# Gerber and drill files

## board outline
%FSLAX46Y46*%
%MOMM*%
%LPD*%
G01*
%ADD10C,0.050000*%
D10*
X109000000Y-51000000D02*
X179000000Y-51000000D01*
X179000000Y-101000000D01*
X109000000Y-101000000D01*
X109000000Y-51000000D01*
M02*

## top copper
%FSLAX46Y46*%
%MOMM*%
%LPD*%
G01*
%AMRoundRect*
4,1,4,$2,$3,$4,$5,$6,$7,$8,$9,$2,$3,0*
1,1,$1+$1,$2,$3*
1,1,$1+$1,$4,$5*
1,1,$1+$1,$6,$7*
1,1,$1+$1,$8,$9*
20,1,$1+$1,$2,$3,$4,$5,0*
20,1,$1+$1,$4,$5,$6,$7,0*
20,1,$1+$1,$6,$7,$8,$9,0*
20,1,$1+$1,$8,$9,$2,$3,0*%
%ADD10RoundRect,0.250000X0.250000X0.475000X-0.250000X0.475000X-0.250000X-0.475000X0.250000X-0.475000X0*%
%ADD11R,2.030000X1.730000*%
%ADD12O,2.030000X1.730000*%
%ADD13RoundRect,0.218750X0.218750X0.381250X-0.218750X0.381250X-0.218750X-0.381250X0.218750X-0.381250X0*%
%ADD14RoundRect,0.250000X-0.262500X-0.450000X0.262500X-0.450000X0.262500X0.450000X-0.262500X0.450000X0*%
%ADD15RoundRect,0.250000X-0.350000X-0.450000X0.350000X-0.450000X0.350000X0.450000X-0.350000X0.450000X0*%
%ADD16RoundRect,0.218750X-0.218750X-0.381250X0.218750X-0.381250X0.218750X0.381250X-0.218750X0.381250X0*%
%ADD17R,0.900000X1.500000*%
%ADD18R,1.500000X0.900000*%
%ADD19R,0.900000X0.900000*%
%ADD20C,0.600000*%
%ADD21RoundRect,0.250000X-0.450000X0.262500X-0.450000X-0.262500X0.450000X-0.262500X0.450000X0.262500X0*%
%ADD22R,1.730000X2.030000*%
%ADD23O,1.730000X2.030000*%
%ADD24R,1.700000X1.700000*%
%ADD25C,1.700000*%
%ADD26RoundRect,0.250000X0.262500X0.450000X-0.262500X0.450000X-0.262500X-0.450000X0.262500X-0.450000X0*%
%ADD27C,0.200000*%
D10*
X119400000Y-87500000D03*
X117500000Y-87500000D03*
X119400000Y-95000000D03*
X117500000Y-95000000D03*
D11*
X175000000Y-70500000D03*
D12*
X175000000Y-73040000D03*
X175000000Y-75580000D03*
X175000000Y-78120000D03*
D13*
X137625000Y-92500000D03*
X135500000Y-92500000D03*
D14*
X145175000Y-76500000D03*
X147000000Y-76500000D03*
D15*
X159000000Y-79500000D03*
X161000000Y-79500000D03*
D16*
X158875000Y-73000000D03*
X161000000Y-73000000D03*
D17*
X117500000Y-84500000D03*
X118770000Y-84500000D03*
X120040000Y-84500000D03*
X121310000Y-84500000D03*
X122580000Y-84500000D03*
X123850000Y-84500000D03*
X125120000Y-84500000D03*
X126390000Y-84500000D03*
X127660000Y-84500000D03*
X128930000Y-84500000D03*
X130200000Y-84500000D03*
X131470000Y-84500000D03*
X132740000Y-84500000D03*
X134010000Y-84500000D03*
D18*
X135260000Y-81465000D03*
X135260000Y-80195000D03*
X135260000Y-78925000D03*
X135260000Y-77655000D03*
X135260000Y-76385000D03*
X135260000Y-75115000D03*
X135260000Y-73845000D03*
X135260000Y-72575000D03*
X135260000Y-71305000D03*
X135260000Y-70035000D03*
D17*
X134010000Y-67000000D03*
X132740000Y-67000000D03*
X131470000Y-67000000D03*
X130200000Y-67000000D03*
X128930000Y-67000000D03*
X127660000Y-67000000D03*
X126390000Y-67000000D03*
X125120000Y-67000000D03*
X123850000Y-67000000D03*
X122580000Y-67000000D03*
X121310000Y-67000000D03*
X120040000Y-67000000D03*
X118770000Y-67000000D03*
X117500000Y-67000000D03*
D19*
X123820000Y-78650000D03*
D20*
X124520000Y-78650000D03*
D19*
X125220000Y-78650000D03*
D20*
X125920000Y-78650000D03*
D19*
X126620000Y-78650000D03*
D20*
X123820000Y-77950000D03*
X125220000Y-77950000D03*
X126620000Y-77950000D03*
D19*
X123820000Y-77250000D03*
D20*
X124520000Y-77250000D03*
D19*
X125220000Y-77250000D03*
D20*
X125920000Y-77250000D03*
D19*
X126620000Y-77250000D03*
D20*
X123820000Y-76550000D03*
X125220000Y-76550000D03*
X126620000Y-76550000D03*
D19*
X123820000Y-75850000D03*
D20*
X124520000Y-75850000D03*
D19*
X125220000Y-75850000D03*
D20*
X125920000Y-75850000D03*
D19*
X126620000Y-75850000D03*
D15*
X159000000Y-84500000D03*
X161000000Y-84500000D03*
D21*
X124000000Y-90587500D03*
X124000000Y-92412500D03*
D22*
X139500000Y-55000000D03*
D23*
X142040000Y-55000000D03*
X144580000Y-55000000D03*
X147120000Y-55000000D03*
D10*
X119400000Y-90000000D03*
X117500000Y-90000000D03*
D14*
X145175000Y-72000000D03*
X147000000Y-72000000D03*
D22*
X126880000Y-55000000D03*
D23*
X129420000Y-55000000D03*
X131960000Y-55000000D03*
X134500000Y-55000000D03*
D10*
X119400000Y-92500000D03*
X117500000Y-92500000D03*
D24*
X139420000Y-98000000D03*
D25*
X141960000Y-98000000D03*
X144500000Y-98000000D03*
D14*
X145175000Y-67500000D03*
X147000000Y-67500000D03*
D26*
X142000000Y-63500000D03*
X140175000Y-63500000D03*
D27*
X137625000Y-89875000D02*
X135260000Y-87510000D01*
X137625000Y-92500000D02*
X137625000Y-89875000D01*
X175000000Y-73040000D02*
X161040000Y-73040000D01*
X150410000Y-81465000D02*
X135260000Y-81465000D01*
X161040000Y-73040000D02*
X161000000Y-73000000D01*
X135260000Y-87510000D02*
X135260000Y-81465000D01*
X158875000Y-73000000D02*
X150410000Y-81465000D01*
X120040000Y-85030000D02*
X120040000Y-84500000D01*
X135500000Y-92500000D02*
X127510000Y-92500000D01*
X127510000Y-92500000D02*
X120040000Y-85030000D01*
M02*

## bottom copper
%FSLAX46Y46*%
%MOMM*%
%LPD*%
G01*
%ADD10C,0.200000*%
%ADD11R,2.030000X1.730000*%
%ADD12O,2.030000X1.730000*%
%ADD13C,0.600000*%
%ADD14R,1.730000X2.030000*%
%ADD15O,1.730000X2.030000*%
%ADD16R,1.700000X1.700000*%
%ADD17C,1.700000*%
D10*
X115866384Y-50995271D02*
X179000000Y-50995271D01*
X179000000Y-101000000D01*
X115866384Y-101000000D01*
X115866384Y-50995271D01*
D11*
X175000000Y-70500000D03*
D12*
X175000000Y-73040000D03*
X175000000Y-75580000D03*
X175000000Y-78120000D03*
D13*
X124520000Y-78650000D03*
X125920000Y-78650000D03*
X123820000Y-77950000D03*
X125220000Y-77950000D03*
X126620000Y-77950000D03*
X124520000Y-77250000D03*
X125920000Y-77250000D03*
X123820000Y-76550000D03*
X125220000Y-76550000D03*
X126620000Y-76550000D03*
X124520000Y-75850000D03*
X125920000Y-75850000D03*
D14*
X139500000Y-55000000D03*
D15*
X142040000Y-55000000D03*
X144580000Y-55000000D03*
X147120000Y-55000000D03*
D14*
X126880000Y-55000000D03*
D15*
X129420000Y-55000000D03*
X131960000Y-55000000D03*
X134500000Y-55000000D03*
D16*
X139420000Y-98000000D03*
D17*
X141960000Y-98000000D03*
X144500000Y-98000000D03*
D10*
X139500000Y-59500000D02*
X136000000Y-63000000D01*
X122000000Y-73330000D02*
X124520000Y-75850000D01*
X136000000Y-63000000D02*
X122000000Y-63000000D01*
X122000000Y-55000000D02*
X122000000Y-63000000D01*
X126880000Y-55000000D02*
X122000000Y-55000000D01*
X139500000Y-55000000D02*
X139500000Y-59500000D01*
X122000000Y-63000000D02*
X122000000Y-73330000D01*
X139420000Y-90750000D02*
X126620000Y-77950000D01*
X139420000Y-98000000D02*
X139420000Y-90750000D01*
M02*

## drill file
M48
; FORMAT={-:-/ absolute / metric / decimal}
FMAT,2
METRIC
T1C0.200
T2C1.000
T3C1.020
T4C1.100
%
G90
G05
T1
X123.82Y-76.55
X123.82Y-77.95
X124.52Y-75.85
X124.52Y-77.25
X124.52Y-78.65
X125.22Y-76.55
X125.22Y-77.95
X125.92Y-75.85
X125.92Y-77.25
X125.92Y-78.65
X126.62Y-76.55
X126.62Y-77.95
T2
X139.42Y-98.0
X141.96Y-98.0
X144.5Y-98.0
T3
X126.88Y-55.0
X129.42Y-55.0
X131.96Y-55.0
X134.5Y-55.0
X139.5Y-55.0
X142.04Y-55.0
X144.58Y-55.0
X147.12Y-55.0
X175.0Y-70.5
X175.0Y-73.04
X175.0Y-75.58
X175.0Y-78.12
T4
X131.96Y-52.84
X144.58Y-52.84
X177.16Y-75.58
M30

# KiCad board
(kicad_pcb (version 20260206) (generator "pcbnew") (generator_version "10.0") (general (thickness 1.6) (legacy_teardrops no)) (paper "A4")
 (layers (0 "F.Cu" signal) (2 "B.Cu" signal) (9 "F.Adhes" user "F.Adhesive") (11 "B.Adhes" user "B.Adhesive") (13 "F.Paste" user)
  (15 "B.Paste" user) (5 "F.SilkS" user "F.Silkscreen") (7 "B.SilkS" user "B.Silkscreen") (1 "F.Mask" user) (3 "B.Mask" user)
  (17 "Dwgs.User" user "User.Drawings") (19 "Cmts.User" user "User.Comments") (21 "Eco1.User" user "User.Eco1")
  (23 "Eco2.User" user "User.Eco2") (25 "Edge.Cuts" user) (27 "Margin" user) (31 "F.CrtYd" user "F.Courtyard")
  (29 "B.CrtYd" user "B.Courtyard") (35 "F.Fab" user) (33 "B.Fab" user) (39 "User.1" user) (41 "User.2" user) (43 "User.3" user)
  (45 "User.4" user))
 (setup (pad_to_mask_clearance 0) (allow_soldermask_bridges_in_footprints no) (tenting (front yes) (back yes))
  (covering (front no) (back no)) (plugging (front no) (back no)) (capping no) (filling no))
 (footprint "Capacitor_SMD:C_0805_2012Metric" (layer "F.Cu") (at 118.45 87.5 180)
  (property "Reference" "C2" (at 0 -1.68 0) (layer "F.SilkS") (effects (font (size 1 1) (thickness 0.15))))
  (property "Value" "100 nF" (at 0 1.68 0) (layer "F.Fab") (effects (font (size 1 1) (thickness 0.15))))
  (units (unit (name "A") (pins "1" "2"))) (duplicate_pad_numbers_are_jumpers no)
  (pad "1" smd roundrect (at -0.95 0 180) (size 1 1.45) (layers "F.Cu" "F.Mask" "F.Paste") (roundrect_rratio 0.25) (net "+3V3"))
  (pad "2" smd roundrect (at 0.95 0 180) (size 1 1.45) (layers "F.Cu" "F.Mask" "F.Paste") (roundrect_rratio 0.25) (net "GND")))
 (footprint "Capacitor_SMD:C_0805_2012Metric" (layer "F.Cu") (at 118.45 95 180)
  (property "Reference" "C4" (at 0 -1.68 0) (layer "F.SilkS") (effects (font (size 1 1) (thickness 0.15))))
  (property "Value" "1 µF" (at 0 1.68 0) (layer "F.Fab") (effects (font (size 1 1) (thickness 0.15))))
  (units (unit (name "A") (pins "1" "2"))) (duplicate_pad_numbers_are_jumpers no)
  (pad "1" smd roundrect (at -0.95 0 180) (size 1 1.45) (layers "F.Cu" "F.Mask" "F.Paste") (roundrect_rratio 0.25) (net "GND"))
  (pad "2" smd roundrect (at 0.95 0 180) (size 1 1.45) (layers "F.Cu" "F.Mask" "F.Paste") (roundrect_rratio 0.25) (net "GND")))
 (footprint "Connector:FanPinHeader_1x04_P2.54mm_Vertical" (layer "F.Cu") (at 175 70.5 -90)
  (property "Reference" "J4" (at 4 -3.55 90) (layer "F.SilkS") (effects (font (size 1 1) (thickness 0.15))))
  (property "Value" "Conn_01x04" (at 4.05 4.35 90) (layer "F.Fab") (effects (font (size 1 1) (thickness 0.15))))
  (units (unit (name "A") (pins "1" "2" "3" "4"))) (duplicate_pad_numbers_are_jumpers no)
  (pad "" np_thru_hole circle (at 5.08 -2.16) (size 1.1 1.1) (drill 1.1) (layers "*.Cu" "*.Mask"))
  (pad "1" thru_hole rect (at 0 0) (size 2.03 1.73) (drill 1.02) (layers "*.Cu" "*.Mask") (remove_unused_layers no) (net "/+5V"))
  (pad "2" thru_hole oval (at 2.54 0) (size 2.03 1.73) (drill 1.02) (layers "*.Cu" "*.Mask") (remove_unused_layers no) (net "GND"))
  (pad "3" thru_hole oval (at 5.08 0) (size 2.03 1.73) (drill 1.02) (layers "*.Cu" "*.Mask") (remove_unused_layers no)
   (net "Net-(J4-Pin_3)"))
  (pad "4" thru_hole oval (at 7.62 0) (size 2.03 1.73) (drill 1.02) (layers "*.Cu" "*.Mask") (remove_unused_layers no) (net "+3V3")))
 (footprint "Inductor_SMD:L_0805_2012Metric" (layer "F.Cu") (at 136.5625 92.5 180)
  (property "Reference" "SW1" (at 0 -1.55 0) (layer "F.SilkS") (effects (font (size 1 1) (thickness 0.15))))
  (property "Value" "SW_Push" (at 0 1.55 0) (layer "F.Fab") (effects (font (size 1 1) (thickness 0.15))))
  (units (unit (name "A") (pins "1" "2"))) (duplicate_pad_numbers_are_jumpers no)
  (pad "1" smd roundrect (at -1.0625 0 180) (size 0.875 1.2) (layers "F.Cu" "F.Mask" "F.Paste") (roundrect_rratio 0.25) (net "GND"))
  (pad "2" smd roundrect (at 1.0625 0 180) (size 0.875 1.2) (layers "F.Cu" "F.Mask" "F.Paste") (roundrect_rratio 0.25) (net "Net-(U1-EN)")))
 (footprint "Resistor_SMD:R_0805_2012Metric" (layer "F.Cu") (at 146.0875 76.5)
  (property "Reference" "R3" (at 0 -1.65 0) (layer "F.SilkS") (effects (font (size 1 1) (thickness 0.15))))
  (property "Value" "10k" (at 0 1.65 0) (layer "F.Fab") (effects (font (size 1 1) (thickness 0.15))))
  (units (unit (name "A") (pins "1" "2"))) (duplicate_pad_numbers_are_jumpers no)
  (pad "1" smd roundrect (at -0.9125 0) (size 1.025 1.4) (layers "F.Cu" "F.Mask" "F.Paste") (roundrect_rratio 0.243902) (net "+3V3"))
  (pad "2" smd roundrect (at 0.9125 0) (size 1.025 1.4) (layers "F.Cu" "F.Mask" "F.Paste") (roundrect_rratio 0.243902) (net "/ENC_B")))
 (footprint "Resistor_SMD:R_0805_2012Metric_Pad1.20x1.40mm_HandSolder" (layer "F.Cu") (at 160 79.5)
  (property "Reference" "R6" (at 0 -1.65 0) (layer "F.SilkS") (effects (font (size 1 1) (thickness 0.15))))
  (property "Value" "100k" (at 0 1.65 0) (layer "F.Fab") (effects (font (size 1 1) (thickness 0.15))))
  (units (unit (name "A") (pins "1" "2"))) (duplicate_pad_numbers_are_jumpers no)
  (pad "1" smd roundrect (at -1 0) (size 1.2 1.4) (layers "F.Cu" "F.Mask" "F.Paste") (roundrect_rratio 0.208333) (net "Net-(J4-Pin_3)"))
  (pad "2" smd roundrect (at 1 0) (size 1.2 1.4) (layers "F.Cu" "F.Mask" "F.Paste") (roundrect_rratio 0.208333) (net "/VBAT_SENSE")))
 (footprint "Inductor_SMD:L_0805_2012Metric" (layer "F.Cu") (at 159.9375 73)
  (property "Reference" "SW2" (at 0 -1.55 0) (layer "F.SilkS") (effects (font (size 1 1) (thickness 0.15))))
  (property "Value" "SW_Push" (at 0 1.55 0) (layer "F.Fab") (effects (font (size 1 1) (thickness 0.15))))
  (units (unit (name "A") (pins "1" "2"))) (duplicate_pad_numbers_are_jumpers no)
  (pad "1" smd roundrect (at -1.0625 0) (size 0.875 1.2) (layers "F.Cu" "F.Mask" "F.Paste") (roundrect_rratio 0.25) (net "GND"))
  (pad "2" smd roundrect (at 1.0625 0) (size 0.875 1.2) (layers "F.Cu" "F.Mask" "F.Paste") (roundrect_rratio 0.25) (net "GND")))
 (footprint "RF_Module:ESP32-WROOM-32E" (layer "F.Cu") (at 122.76 75.75 90)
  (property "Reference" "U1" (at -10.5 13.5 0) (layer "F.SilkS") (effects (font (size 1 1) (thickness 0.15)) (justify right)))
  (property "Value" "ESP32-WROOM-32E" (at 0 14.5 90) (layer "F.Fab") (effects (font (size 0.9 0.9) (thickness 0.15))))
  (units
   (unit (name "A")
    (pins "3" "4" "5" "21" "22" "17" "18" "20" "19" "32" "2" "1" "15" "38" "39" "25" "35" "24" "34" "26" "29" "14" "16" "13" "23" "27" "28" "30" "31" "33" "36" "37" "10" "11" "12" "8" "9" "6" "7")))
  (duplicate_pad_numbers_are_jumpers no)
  (pad "1" smd rect (at -8.75 -5.26 90) (size 1.5 0.9) (layers "F.Cu" "F.Mask" "F.Paste") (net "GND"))
  (pad "2" smd rect (at -8.75 -3.99 90) (size 1.5 0.9) (layers "F.Cu" "F.Mask" "F.Paste") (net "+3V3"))
  (pad "3" smd rect (at -8.75 -2.72 90) (size 1.5 0.9) (layers "F.Cu" "F.Mask" "F.Paste") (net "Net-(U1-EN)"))
  (pad "4" smd rect (at -8.75 -1.45 90) (size 1.5 0.9) (layers "F.Cu" "F.Mask" "F.Paste") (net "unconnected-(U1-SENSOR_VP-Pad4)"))
  (pad "5" smd rect (at -8.75 -0.18 90) (size 1.5 0.9) (layers "F.Cu" "F.Mask" "F.Paste") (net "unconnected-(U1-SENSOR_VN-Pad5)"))
  (pad "6" smd rect (at -8.75 1.09 90) (size 1.5 0.9) (layers "F.Cu" "F.Mask" "F.Paste") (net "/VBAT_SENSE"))
  (pad "7" smd rect (at -8.75 2.36 90) (size 1.5 0.9) (layers "F.Cu" "F.Mask" "F.Paste") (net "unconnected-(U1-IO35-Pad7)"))
  (pad "8" smd rect (at -8.75 3.63 90) (size 1.5 0.9) (layers "F.Cu" "F.Mask" "F.Paste") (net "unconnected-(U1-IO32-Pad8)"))
  (pad "9" smd rect (at -8.75 4.9 90) (size 1.5 0.9) (layers "F.Cu" "F.Mask" "F.Paste") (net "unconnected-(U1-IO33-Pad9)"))
  (pad "10" smd rect (at -8.75 6.17 90) (size 1.5 0.9) (layers "F.Cu" "F.Mask" "F.Paste") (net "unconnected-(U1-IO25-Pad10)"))
  (pad "11" smd rect (at -8.75 7.44 90) (size 1.5 0.9) (layers "F.Cu" "F.Mask" "F.Paste") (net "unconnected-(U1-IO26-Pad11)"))
  (pad "12" smd rect (at -8.75 8.71 90) (size 1.5 0.9) (layers "F.Cu" "F.Mask" "F.Paste") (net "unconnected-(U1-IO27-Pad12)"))
  (pad "13" smd rect (at -8.75 9.98 90) (size 1.5 0.9) (layers "F.Cu" "F.Mask" "F.Paste") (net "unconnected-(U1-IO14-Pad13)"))
  (pad "14" smd rect (at -8.75 11.25 90) (size 1.5 0.9) (layers "F.Cu" "F.Mask" "F.Paste") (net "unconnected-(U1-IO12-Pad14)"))
  (pad "15" smd rect (at -5.715 12.5 180) (size 1.5 0.9) (layers "F.Cu" "F.Mask" "F.Paste") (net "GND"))
  (pad "16" smd rect (at -4.445 12.5 180) (size 1.5 0.9) (layers "F.Cu" "F.Mask" "F.Paste") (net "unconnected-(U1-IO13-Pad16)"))
  (pad "17" smd rect (at -3.175 12.5 180) (size 1.5 0.9) (layers "F.Cu" "F.Mask" "F.Paste") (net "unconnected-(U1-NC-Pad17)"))
  (pad "18" smd rect (at -1.905 12.5 180) (size 1.5 0.9) (layers "F.Cu" "F.Mask" "F.Paste") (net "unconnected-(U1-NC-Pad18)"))
  (pad "19" smd rect (at -0.635 12.5 180) (size 1.5 0.9) (layers "F.Cu" "F.Mask" "F.Paste") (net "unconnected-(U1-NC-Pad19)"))
  (pad "20" smd rect (at 0.635 12.5 180) (size 1.5 0.9) (layers "F.Cu" "F.Mask" "F.Paste") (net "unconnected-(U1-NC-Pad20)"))
  (pad "21" smd rect (at 1.905 12.5 180) (size 1.5 0.9) (layers "F.Cu" "F.Mask" "F.Paste") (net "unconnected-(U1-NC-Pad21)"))
  (pad "22" smd rect (at 3.175 12.5 180) (size 1.5 0.9) (layers "F.Cu" "F.Mask" "F.Paste") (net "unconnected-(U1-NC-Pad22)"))
  (pad "23" smd rect (at 4.445 12.5 180) (size 1.5 0.9) (layers "F.Cu" "F.Mask" "F.Paste") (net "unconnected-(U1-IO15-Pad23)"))
  (pad "24" smd rect (at 5.715 12.5 180) (size 1.5 0.9) (layers "F.Cu" "F.Mask" "F.Paste") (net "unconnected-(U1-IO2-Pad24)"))
  (pad "25" smd rect (at 8.75 11.25 90) (size 1.5 0.9) (layers "F.Cu" "F.Mask" "F.Paste") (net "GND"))
  (pad "26" smd rect (at 8.75 9.98 90) (size 1.5 0.9) (layers "F.Cu" "F.Mask" "F.Paste") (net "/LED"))
  (pad "27" smd rect (at 8.75 8.71 90) (size 1.5 0.9) (layers "F.Cu" "F.Mask" "F.Paste") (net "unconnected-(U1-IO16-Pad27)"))
  (pad "28" smd rect (at 8.75 7.44 90) (size 1.5 0.9) (layers "F.Cu" "F.Mask" "F.Paste") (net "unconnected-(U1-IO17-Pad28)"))
  (pad "29" smd rect (at 8.75 6.17 90) (size 1.5 0.9) (layers "F.Cu" "F.Mask" "F.Paste") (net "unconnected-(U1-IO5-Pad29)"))
  (pad "30" smd rect (at 8.75 4.9 90) (size 1.5 0.9) (layers "F.Cu" "F.Mask" "F.Paste") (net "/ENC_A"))
  (pad "31" smd rect (at 8.75 3.63 90) (size 1.5 0.9) (layers "F.Cu" "F.Mask" "F.Paste") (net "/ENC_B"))
  (pad "32" smd rect (at 8.75 2.36 90) (size 1.5 0.9) (layers "F.Cu" "F.Mask" "F.Paste") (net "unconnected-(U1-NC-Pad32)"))
  (pad "33" smd rect (at 8.75 1.09 90) (size 1.5 0.9) (layers "F.Cu" "F.Mask" "F.Paste") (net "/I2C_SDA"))
  (pad "34" smd rect (at 8.75 -0.18 90) (size 1.5 0.9) (layers "F.Cu" "F.Mask" "F.Paste") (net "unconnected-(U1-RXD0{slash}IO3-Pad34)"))
  (pad "35" smd rect (at 8.75 -1.45 90) (size 1.5 0.9) (layers "F.Cu" "F.Mask" "F.Paste") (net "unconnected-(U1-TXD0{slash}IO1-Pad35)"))
  (pad "36" smd rect (at 8.75 -2.72 90) (size 1.5 0.9) (layers "F.Cu" "F.Mask" "F.Paste") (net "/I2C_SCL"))
  (pad "37" smd rect (at 8.75 -3.99 90) (size 1.5 0.9) (layers "F.Cu" "F.Mask" "F.Paste") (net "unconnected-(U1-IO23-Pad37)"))
  (pad "38" smd rect (at 8.75 -5.26 90) (size 1.5 0.9) (layers "F.Cu" "F.Mask" "F.Paste") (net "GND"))
  (pad "39" smd rect (at -2.9 1.06 90) (size 0.9 0.9) (layers "F.Cu" "F.Mask" "F.Paste") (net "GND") (zone_connect 2))
  (pad "39" thru_hole circle (at -2.9 1.76 90) (size 0.6 0.6) (drill 0.2) (layers "*.Cu" "*.Mask") (remove_unused_layers no) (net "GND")
   (zone_connect 2))
  (pad "39" smd rect (at -2.9 2.46 90) (size 0.9 0.9) (layers "F.Cu" "F.Mask" "F.Paste") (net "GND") (zone_connect 2))
  (pad "39" thru_hole circle (at -2.9 3.16 90) (size 0.6 0.6) (drill 0.2) (layers "*.Cu" "*.Mask") (remove_unused_layers no) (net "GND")
   (zone_connect 2))
  (pad "39" smd rect (at -2.9 3.86 90) (size 0.9 0.9) (layers "F.Cu" "F.Mask" "F.Paste") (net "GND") (zone_connect 2))
  (pad "39" thru_hole circle (at -2.2 1.06 90) (size 0.6 0.6) (drill 0.2) (layers "*.Cu" "*.Mask") (remove_unused_layers no) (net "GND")
   (zone_connect 2))
  (pad "39" thru_hole circle (at -2.2 2.46 90) (size 0.6 0.6) (drill 0.2) (layers "*.Cu" "*.Mask") (remove_unused_layers no) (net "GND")
   (zone_connect 2))
  (pad "39" thru_hole circle (at -2.2 3.86 90) (size 0.6 0.6) (drill 0.2) (layers "*.Cu" "*.Mask") (remove_unused_layers no) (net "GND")
   (zone_connect 2))
  (pad "39" smd rect (at -1.5 1.06 90) (size 0.9 0.9) (layers "F.Cu" "F.Mask" "F.Paste") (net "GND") (zone_connect 2))
  (pad "39" thru_hole circle (at -1.5 1.76 90) (size 0.6 0.6) (drill 0.2) (layers "*.Cu" "*.Mask") (remove_unused_layers no) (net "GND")
   (zone_connect 2))
  (pad "39" smd rect (at -1.5 2.46 90) (size 0.9 0.9) (layers "F.Cu" "F.Mask" "F.Paste") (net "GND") (zone_connect 2))
  (pad "39" thru_hole circle (at -1.5 3.16 90) (size 0.6 0.6) (drill 0.2) (layers "*.Cu" "*.Mask") (remove_unused_layers no) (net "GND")
   (zone_connect 2))
  (pad "39" smd rect (at -1.5 3.86 90) (size 0.9 0.9) (layers "F.Cu" "F.Mask" "F.Paste") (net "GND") (zone_connect 2))
  (pad "39" thru_hole circle (at -0.8 1.06 90) (size 0.6 0.6) (drill 0.2) (layers "*.Cu" "*.Mask") (remove_unused_layers no) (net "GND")
   (zone_connect 2))
  (pad "39" thru_hole circle (at -0.8 2.46 90) (size 0.6 0.6) (drill 0.2) (layers "*.Cu" "*.Mask") (remove_unused_layers no) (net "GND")
   (zone_connect 2))
  (pad "39" thru_hole circle (at -0.8 3.86 90) (size 0.6 0.6) (drill 0.2) (layers "*.Cu" "*.Mask") (remove_unused_layers no) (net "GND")
   (zone_connect 2))
  (pad "39" smd rect (at -0.1 1.06 90) (size 0.9 0.9) (layers "F.Cu" "F.Mask" "F.Paste") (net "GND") (zone_connect 2))
  (pad "39" thru_hole circle (at -0.1 1.76 90) (size 0.6 0.6) (drill 0.2) (layers "*.Cu" "*.Mask") (remove_unused_layers no) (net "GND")
   (zone_connect 2))
  (pad "39" smd rect (at -0.1 2.46 90) (size 0.9 0.9) (layers "F.Cu" "F.Mask" "F.Paste") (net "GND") (zone_connect 2))
  (pad "39" thru_hole circle (at -0.1 3.16 90) (size 0.6 0.6) (drill 0.2) (layers "*.Cu" "*.Mask") (remove_unused_layers no) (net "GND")
   (zone_connect 2))
  (pad "39" smd rect (at -0.1 3.86 90) (size 0.9 0.9) (layers "F.Cu" "F.Mask" "F.Paste") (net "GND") (zone_connect 2))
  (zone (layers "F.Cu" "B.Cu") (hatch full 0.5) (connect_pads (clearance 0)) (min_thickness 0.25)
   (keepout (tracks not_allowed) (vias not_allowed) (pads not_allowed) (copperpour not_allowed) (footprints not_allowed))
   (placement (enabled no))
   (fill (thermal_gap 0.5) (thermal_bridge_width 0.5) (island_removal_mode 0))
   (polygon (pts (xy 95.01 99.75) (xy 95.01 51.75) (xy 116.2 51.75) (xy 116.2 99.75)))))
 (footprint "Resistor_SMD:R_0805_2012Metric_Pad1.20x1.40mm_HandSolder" (layer "F.Cu") (at 160 84.5)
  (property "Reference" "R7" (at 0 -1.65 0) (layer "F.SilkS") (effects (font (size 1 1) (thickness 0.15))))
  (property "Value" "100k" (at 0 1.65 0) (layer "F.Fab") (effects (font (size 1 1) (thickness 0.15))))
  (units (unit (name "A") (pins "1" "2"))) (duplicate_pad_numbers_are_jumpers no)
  (pad "1" smd roundrect (at -1 0) (size 1.2 1.4) (layers "F.Cu" "F.Mask" "F.Paste") (roundrect_rratio 0.208333) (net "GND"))
  (pad "2" smd roundrect (at 1 0) (size 1.2 1.4) (layers "F.Cu" "F.Mask" "F.Paste") (roundrect_rratio 0.208333) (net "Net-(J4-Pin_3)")))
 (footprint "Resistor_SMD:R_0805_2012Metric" (layer "F.Cu") (at 124 91.5 -90)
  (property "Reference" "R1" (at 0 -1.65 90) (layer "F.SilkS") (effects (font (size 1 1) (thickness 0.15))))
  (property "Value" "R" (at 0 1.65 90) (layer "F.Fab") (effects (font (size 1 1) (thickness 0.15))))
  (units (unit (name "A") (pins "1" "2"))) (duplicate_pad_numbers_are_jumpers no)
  (pad "1" smd roundrect (at -0.9125 0 270) (size 1.025 1.4) (layers "F.Cu" "F.Mask" "F.Paste") (roundrect_rratio 0.243902) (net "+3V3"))
  (pad "2" smd roundrect (at 0.9125 0 270) (size 1.025 1.4) (layers "F.Cu" "F.Mask" "F.Paste") (roundrect_rratio 0.243902)
   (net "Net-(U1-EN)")))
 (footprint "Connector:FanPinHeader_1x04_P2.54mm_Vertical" (layer "F.Cu") (at 139.5 55)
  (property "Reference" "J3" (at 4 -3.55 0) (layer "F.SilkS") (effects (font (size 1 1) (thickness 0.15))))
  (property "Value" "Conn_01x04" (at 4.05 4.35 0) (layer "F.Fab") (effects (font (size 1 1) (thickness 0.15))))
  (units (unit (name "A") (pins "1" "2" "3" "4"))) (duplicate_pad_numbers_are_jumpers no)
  (pad "" np_thru_hole circle (at 5.08 -2.16 90) (size 1.1 1.1) (drill 1.1) (layers "*.Cu" "*.Mask"))
  (pad "1" thru_hole rect (at 0 0 90) (size 2.03 1.73) (drill 1.02) (layers "*.Cu" "*.Mask") (remove_unused_layers no) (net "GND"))
  (pad "2" thru_hole oval (at 2.54 0 90) (size 2.03 1.73) (drill 1.02) (layers "*.Cu" "*.Mask") (remove_unused_layers no) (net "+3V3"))
  (pad "3" thru_hole oval (at 5.08 0 90) (size 2.03 1.73) (drill 1.02) (layers "*.Cu" "*.Mask") (remove_unused_layers no) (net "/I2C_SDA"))
  (pad "4" thru_hole oval (at 7.62 0 90) (size 2.03 1.73) (drill 1.02) (layers "*.Cu" "*.Mask") (remove_unused_layers no) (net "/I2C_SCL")))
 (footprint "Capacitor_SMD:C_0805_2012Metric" (layer "F.Cu") (at 118.45 90 180)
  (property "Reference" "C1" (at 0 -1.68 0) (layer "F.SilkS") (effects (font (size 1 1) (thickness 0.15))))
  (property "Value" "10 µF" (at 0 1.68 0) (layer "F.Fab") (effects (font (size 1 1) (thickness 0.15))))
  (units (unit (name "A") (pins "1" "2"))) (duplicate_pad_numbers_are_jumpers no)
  (pad "1" smd roundrect (at -0.95 0 180) (size 1 1.45) (layers "F.Cu" "F.Mask" "F.Paste") (roundrect_rratio 0.25) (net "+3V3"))
  (pad "2" smd roundrect (at 0.95 0 180) (size 1 1.45) (layers "F.Cu" "F.Mask" "F.Paste") (roundrect_rratio 0.25) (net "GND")))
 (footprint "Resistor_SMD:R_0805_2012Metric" (layer "F.Cu") (at 146.0875 72)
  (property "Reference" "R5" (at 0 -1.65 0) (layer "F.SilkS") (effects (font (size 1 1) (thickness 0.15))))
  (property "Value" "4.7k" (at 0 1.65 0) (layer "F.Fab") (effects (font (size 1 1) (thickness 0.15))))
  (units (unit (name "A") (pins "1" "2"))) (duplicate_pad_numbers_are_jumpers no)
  (pad "1" smd roundrect (at -0.9125 0) (size 1.025 1.4) (layers "F.Cu" "F.Mask" "F.Paste") (roundrect_rratio 0.243902) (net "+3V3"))
  (pad "2" smd roundrect (at 0.9125 0) (size 1.025 1.4) (layers "F.Cu" "F.Mask" "F.Paste") (roundrect_rratio 0.243902) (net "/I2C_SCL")))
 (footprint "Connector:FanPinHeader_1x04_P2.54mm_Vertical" (layer "F.Cu") (at 126.88 55)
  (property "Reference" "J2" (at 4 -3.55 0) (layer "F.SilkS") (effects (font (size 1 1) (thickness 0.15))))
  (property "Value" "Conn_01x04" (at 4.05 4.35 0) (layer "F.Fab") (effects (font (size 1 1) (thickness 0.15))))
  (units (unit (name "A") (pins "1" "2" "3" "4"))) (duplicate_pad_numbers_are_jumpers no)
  (pad "" np_thru_hole circle (at 5.08 -2.16 90) (size 1.1 1.1) (drill 1.1) (layers "*.Cu" "*.Mask"))
  (pad "1" thru_hole rect (at 0 0 90) (size 2.03 1.73) (drill 1.02) (layers "*.Cu" "*.Mask") (remove_unused_layers no) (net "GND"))
  (pad "2" thru_hole oval (at 2.54 0 90) (size 2.03 1.73) (drill 1.02) (layers "*.Cu" "*.Mask") (remove_unused_layers no) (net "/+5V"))
  (pad "3" thru_hole oval (at 5.08 0 90) (size 2.03 1.73) (drill 1.02) (layers "*.Cu" "*.Mask") (remove_unused_layers no) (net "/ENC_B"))
  (pad "4" thru_hole oval (at 7.62 0 90) (size 2.03 1.73) (drill 1.02) (layers "*.Cu" "*.Mask") (remove_unused_layers no) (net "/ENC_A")))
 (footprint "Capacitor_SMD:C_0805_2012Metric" (layer "F.Cu") (at 118.45 92.5 180)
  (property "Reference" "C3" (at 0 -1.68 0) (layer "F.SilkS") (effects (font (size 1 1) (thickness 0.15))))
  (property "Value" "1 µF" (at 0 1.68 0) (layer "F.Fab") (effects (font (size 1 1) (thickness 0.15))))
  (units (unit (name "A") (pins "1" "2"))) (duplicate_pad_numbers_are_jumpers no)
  (pad "1" smd roundrect (at -0.95 0 180) (size 1 1.45) (layers "F.Cu" "F.Mask" "F.Paste") (roundrect_rratio 0.25) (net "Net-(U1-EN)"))
  (pad "2" smd roundrect (at 0.95 0 180) (size 1 1.45) (layers "F.Cu" "F.Mask" "F.Paste") (roundrect_rratio 0.25) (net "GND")))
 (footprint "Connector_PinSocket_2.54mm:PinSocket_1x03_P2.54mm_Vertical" (layer "F.Cu") (at 139.42 98 90)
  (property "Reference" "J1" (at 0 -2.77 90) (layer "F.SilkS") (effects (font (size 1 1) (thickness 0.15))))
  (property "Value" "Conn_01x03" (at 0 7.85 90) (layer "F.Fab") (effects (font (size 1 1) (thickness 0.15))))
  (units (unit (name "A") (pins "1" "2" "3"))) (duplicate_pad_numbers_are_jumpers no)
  (pad "1" thru_hole rect (at 0 0 90) (size 1.7 1.7) (drill 1) (layers "*.Cu" "*.Mask") (remove_unused_layers no) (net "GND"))
  (pad "2" thru_hole circle (at 0 2.54 90) (size 1.7 1.7) (drill 1) (layers "*.Cu" "*.Mask") (remove_unused_layers no) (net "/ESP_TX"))
  (pad "3" thru_hole circle (at 0 5.08 90) (size 1.7 1.7) (drill 1) (layers "*.Cu" "*.Mask") (remove_unused_layers no) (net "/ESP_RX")))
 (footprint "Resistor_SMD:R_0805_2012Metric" (layer "F.Cu") (at 146.0875 67.5)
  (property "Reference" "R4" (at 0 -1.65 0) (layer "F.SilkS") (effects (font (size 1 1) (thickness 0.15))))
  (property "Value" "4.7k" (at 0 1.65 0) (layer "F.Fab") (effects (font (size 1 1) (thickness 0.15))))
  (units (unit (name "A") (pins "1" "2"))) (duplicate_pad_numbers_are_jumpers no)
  (pad "1" smd roundrect (at -0.9125 0) (size 1.025 1.4) (layers "F.Cu" "F.Mask" "F.Paste") (roundrect_rratio 0.243902) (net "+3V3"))
  (pad "2" smd roundrect (at 0.9125 0) (size 1.025 1.4) (layers "F.Cu" "F.Mask" "F.Paste") (roundrect_rratio 0.243902) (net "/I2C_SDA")))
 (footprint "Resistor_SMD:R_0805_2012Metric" (layer "F.Cu") (at 141.0875 63.5 180)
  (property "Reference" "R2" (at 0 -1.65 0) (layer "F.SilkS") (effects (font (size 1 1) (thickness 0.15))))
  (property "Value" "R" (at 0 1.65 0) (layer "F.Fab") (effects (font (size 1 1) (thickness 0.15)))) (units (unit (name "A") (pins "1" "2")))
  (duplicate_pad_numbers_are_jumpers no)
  (pad "1" smd roundrect (at -0.9125 0 180) (size 1.025 1.4) (layers "F.Cu" "F.Mask" "F.Paste") (roundrect_rratio 0.243902) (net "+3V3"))
  (pad "2" smd roundrect (at 0.9125 0 180) (size 1.025 1.4) (layers "F.Cu" "F.Mask" "F.Paste") (roundrect_rratio 0.243902) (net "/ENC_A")))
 (gr_rect (start 115.866384 50.995271) (end 179 101) (stroke (width 0.2) (type default)) (fill no) (layer "B.Cu") (net "GND"))
 (gr_rect (start 109 51) (end 179 101) (stroke (width 0.05) (type default)) (fill no) (layer "Edge.Cuts"))
 (segment (start 137.625 89.875) (end 135.26 87.51) (width 0.2) (layer "F.Cu") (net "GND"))
 (segment (start 137.625 92.5) (end 137.625 89.875) (width 0.2) (layer "F.Cu") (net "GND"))
 (segment (start 175 73.04) (end 161.04 73.04) (width 0.2) (layer "F.Cu") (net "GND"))
 (segment (start 150.41 81.465) (end 135.26 81.465) (width 0.2) (layer "F.Cu") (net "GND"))
 (segment (start 161.04 73.04) (end 161 73) (width 0.2) (layer "F.Cu") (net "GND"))
 (segment (start 135.26 87.51) (end 135.26 81.465) (width 0.2) (layer "F.Cu") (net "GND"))
 (segment (start 158.875 73) (end 150.41 81.465) (width 0.2) (layer "F.Cu") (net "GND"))
 (segment (start 139.5 59.5) (end 136 63) (width 0.2) (layer "B.Cu") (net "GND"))
 (segment (start 122 73.33) (end 124.52 75.85) (width 0.2) (layer "B.Cu") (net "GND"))
 (segment (start 136 63) (end 122 63) (width 0.2) (layer "B.Cu") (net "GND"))
 (segment (start 122 55) (end 122 63) (width 0.2) (layer "B.Cu") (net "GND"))
 (segment (start 126.88 55) (end 122 55) (width 0.2) (layer "B.Cu") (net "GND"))
 (segment (start 139.5 55) (end 139.5 59.5) (width 0.2) (layer "B.Cu") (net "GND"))
 (segment (start 122 63) (end 122 73.33) (width 0.2) (layer "B.Cu") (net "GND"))
 (segment (start 139.42 90.75) (end 126.62 77.95) (width 0.2) (layer "B.Cu") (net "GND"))
 (segment (start 139.42 98) (end 139.42 90.75) (width 0.2) (layer "B.Cu") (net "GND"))
 (segment (start 120.04 85.03) (end 120.04 84.5) (width 0.2) (layer "F.Cu") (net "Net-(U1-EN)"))
 (segment (start 135.5 92.5) (end 127.51 92.5) (width 0.2) (layer "F.Cu") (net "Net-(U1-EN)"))
 (segment (start 127.51 92.5) (end 120.04 85.03) (width 0.2) (layer "F.Cu") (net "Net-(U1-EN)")))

